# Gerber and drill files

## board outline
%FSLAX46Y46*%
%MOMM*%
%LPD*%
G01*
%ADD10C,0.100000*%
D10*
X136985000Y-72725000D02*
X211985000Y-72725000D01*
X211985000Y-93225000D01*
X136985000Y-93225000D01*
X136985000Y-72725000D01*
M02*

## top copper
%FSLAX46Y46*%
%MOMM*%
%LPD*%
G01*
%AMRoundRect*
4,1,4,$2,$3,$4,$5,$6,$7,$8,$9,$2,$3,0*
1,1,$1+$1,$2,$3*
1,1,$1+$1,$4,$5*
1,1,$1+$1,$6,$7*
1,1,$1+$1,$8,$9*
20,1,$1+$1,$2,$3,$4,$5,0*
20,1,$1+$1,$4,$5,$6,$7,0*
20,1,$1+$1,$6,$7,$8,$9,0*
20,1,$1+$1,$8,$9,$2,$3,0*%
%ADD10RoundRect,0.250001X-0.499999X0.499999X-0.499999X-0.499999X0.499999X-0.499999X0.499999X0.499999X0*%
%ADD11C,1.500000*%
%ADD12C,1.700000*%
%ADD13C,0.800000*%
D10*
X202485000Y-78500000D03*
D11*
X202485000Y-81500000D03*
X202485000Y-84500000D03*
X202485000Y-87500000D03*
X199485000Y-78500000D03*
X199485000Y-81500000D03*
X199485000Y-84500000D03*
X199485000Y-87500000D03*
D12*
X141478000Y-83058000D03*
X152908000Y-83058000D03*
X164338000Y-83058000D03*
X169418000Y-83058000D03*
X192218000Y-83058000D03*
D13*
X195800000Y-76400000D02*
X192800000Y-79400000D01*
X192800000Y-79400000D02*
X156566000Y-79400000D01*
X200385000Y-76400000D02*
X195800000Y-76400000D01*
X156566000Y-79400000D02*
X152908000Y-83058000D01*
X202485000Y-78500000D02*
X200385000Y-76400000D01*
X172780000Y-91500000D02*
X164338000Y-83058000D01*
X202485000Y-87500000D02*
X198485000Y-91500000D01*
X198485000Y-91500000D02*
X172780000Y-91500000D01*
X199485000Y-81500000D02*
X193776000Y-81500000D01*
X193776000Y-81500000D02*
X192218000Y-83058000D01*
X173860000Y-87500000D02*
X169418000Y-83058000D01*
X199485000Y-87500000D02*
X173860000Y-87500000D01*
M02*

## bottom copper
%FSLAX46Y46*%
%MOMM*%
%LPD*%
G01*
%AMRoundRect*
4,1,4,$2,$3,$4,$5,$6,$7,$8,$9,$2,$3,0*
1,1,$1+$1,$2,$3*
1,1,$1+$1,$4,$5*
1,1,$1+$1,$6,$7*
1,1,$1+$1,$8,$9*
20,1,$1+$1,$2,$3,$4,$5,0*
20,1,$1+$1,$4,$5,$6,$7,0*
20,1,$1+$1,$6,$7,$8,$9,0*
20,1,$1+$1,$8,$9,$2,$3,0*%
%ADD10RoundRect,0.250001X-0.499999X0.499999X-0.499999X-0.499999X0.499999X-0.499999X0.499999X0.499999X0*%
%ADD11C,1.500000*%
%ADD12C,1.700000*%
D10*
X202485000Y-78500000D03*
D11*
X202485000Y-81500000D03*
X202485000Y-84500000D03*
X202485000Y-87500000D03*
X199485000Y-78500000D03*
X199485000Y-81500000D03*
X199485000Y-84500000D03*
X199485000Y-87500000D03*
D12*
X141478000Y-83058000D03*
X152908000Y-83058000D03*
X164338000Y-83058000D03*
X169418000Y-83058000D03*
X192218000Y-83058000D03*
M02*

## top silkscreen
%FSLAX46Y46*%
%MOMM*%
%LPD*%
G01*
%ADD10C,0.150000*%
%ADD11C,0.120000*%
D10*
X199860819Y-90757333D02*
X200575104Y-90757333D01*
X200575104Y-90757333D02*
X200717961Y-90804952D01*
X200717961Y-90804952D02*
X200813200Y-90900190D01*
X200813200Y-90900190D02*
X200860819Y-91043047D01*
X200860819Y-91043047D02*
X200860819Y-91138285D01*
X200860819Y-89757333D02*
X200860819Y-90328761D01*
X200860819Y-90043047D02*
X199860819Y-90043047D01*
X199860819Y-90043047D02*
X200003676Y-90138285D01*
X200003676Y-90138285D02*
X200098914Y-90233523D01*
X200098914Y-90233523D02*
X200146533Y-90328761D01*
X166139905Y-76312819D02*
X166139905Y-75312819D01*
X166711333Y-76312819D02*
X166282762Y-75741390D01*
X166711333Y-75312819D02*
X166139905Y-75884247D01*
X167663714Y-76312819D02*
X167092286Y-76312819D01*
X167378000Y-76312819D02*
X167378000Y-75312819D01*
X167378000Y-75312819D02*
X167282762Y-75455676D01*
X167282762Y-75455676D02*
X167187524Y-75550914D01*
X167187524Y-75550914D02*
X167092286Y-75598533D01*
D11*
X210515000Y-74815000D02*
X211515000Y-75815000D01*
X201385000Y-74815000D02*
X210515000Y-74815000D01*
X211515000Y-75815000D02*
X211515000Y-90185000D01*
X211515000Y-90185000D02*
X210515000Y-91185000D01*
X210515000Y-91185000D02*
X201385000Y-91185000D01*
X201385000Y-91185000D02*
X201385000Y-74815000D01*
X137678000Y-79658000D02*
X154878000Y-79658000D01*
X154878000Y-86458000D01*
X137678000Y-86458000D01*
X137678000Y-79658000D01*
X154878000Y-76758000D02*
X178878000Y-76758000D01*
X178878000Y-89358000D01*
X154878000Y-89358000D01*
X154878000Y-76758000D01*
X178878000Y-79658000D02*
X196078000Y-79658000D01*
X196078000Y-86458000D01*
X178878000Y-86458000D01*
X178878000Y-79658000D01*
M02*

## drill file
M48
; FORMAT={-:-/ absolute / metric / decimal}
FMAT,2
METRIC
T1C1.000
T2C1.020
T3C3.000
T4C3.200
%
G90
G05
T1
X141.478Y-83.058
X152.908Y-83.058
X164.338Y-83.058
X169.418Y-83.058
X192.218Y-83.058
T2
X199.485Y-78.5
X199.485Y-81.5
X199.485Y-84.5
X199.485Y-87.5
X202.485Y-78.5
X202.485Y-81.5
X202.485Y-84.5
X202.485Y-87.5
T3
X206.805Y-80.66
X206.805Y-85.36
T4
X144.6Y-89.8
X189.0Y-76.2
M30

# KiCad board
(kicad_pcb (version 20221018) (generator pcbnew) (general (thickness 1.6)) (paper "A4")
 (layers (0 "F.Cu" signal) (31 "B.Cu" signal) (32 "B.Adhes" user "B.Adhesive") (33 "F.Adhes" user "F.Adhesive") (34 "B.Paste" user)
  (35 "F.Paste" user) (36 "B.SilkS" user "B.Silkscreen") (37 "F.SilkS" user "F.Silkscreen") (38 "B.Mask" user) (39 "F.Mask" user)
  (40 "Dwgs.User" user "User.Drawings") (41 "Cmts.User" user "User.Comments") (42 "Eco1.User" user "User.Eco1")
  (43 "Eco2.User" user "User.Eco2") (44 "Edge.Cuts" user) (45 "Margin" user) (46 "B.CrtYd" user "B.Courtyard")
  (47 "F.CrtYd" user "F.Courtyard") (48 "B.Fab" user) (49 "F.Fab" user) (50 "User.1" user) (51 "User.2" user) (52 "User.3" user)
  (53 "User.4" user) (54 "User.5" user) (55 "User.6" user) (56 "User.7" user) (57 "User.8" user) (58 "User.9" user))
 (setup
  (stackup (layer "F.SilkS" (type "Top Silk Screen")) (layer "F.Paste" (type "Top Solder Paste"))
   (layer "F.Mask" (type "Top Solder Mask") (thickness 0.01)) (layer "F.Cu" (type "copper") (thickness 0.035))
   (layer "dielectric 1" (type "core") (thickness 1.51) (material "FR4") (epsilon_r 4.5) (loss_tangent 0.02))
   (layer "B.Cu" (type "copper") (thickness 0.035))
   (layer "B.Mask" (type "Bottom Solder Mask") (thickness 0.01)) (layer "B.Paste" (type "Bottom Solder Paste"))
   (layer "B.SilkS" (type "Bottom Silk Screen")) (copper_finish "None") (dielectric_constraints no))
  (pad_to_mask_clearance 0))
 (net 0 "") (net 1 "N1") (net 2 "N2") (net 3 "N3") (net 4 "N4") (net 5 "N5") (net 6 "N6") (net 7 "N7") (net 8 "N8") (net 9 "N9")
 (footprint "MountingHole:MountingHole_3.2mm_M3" (layer "F.Cu") (at 144.6 89.8)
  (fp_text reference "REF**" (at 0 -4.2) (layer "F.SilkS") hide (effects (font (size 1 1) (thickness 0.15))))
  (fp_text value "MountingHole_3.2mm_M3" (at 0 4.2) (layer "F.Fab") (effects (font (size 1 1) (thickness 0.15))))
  (pad "" np_thru_hole circle (at 0 0) (size 3.2 3.2) (drill 3.2) (layers "*.Cu" "*.Mask")))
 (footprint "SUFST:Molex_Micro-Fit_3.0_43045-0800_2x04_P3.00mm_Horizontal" (layer "F.Cu") (at 202.485 78.5 -90)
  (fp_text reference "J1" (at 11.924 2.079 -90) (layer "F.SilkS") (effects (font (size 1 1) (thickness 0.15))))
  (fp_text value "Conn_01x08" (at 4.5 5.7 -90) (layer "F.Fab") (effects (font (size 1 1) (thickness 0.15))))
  (fp_line (start -3.685 -8.03) (end -2.685 -9.03) (stroke (width 0.12) (type solid)) (layer "F.SilkS"))
  (fp_line (start -3.685 1.1) (end -3.685 -8.03) (stroke (width 0.12) (type solid)) (layer "F.SilkS"))
  (fp_line (start -2.685 -9.03) (end 11.685 -9.03) (stroke (width 0.12) (type solid)) (layer "F.SilkS"))
  (fp_line (start 11.685 -9.03) (end 12.685 -8.03) (stroke (width 0.12) (type solid)) (layer "F.SilkS"))
  (fp_line (start 12.685 -8.03) (end 12.685 1.1) (stroke (width 0.12) (type solid)) (layer "F.SilkS"))
  (fp_line (start 12.685 1.1) (end -3.685 1.1) (stroke (width 0.12) (type solid)) (layer "F.SilkS"))
  (pad "" np_thru_hole circle (at 2.16 -4.32 270) (size 3 3) (drill 3) (layers "*.Cu" "*.Mask"))
  (pad "" np_thru_hole circle (at 6.86 -4.32 270) (size 3 3) (drill 3) (layers "*.Cu" "*.Mask"))
  (pad "1" thru_hole roundrect (at 0 0 270) (size 1.5 1.5) (drill 1.02) (layers "*.Cu" "*.Mask") (roundrect_rratio 0.166667) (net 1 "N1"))
  (pad "2" thru_hole circle (at 3 0 270) (size 1.5 1.5) (drill 1.02) (layers "*.Cu" "*.Mask") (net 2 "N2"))
  (pad "3" thru_hole circle (at 6 0 270) (size 1.5 1.5) (drill 1.02) (layers "*.Cu" "*.Mask") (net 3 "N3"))
  (pad "4" thru_hole circle (at 9 0 270) (size 1.5 1.5) (drill 1.02) (layers "*.Cu" "*.Mask") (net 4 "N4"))
  (pad "5" thru_hole circle (at 0 3 270) (size 1.5 1.5) (drill 1.02) (layers "*.Cu" "*.Mask") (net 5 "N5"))
  (pad "6" thru_hole circle (at 3 3 270) (size 1.5 1.5) (drill 1.02) (layers "*.Cu" "*.Mask") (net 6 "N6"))
  (pad "7" thru_hole circle (at 6 3 270) (size 1.5 1.5) (drill 1.02) (layers "*.Cu" "*.Mask") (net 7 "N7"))
  (pad "8" thru_hole circle (at 9 3 270) (size 1.5 1.5) (drill 1.02) (layers "*.Cu" "*.Mask") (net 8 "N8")))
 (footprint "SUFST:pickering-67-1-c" (layer "F.Cu") (at 166.878 83.058)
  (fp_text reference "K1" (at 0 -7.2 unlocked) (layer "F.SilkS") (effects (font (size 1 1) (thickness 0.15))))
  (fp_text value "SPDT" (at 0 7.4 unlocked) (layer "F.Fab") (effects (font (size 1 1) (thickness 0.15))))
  (fp_rect (start -29.2 -3.4) (end -12 3.4) (stroke (width 0.12) (type solid)) (fill none) (layer "F.SilkS"))
  (fp_rect (start -12 -6.3) (end 12 6.3) (stroke (width 0.12) (type solid)) (fill none) (layer "F.SilkS"))
  (fp_rect (start 12 -3.4) (end 29.2 3.4) (stroke (width 0.12) (type solid)) (fill none) (layer "F.SilkS"))
  (pad "1" thru_hole circle (at -25.4 0) (size 1.7 1.7) (drill 1) (layers "*.Cu" "*.Mask") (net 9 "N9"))
  (pad "2" thru_hole circle (at -13.97 0) (size 1.7 1.7) (drill 1) (layers "*.Cu" "*.Mask") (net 1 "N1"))
  (pad "3" thru_hole circle (at -2.54 0) (size 1.7 1.7) (drill 1) (layers "*.Cu" "*.Mask") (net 4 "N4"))
  (pad "5" thru_hole circle (at 2.54 0) (size 1.7 1.7) (drill 1) (layers "*.Cu" "*.Mask") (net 8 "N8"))
  (pad "7" thru_hole circle (at 25.34 0) (size 1.7 1.7) (drill 1) (layers "*.Cu" "*.Mask") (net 6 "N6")))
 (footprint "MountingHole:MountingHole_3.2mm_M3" (layer "F.Cu") (at 189 76.2)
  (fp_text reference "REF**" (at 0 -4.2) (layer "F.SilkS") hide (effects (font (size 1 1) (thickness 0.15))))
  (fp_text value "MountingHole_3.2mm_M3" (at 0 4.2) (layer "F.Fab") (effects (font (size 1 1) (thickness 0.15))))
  (pad "" np_thru_hole circle (at 0 0) (size 3.2 3.2) (drill 3.2) (layers "*.Cu" "*.Mask")))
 (gr_rect (start 136.985 72.725) (end 211.985 93.225) (stroke (width 0.1) (type solid)) (fill none) (layer "Edge.Cuts"))
 (segment (start 195.8 76.4) (end 192.8 79.4) (width 0.8) (layer "F.Cu") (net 1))
 (segment (start 192.8 79.4) (end 156.566 79.4) (width 0.8) (layer "F.Cu") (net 1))
 (segment (start 200.385 76.4) (end 195.8 76.4) (width 0.8) (layer "F.Cu") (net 1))
 (segment (start 156.566 79.4) (end 152.908 83.058) (width 0.8) (layer "F.Cu") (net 1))
 (segment (start 202.485 78.5) (end 200.385 76.4) (width 0.8) (layer "F.Cu") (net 1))
 (segment (start 172.78 91.5) (end 164.338 83.058) (width 0.8) (layer "F.Cu") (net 4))
 (segment (start 202.485 87.5) (end 198.485 91.5) (width 0.8) (layer "F.Cu") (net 4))
 (segment (start 198.485 91.5) (end 172.78 91.5) (width 0.8) (layer "F.Cu") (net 4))
 (segment (start 199.485 81.5) (end 193.776 81.5) (width 0.8) (layer "F.Cu") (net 6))
 (segment (start 193.776 81.5) (end 192.218 83.058) (width 0.8) (layer "F.Cu") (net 6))
 (segment (start 173.86 87.5) (end 169.418 83.058) (width 0.8) (layer "F.Cu") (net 8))
 (segment (start 199.485 87.5) (end 173.86 87.5) (width 0.8) (layer "F.Cu") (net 8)))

